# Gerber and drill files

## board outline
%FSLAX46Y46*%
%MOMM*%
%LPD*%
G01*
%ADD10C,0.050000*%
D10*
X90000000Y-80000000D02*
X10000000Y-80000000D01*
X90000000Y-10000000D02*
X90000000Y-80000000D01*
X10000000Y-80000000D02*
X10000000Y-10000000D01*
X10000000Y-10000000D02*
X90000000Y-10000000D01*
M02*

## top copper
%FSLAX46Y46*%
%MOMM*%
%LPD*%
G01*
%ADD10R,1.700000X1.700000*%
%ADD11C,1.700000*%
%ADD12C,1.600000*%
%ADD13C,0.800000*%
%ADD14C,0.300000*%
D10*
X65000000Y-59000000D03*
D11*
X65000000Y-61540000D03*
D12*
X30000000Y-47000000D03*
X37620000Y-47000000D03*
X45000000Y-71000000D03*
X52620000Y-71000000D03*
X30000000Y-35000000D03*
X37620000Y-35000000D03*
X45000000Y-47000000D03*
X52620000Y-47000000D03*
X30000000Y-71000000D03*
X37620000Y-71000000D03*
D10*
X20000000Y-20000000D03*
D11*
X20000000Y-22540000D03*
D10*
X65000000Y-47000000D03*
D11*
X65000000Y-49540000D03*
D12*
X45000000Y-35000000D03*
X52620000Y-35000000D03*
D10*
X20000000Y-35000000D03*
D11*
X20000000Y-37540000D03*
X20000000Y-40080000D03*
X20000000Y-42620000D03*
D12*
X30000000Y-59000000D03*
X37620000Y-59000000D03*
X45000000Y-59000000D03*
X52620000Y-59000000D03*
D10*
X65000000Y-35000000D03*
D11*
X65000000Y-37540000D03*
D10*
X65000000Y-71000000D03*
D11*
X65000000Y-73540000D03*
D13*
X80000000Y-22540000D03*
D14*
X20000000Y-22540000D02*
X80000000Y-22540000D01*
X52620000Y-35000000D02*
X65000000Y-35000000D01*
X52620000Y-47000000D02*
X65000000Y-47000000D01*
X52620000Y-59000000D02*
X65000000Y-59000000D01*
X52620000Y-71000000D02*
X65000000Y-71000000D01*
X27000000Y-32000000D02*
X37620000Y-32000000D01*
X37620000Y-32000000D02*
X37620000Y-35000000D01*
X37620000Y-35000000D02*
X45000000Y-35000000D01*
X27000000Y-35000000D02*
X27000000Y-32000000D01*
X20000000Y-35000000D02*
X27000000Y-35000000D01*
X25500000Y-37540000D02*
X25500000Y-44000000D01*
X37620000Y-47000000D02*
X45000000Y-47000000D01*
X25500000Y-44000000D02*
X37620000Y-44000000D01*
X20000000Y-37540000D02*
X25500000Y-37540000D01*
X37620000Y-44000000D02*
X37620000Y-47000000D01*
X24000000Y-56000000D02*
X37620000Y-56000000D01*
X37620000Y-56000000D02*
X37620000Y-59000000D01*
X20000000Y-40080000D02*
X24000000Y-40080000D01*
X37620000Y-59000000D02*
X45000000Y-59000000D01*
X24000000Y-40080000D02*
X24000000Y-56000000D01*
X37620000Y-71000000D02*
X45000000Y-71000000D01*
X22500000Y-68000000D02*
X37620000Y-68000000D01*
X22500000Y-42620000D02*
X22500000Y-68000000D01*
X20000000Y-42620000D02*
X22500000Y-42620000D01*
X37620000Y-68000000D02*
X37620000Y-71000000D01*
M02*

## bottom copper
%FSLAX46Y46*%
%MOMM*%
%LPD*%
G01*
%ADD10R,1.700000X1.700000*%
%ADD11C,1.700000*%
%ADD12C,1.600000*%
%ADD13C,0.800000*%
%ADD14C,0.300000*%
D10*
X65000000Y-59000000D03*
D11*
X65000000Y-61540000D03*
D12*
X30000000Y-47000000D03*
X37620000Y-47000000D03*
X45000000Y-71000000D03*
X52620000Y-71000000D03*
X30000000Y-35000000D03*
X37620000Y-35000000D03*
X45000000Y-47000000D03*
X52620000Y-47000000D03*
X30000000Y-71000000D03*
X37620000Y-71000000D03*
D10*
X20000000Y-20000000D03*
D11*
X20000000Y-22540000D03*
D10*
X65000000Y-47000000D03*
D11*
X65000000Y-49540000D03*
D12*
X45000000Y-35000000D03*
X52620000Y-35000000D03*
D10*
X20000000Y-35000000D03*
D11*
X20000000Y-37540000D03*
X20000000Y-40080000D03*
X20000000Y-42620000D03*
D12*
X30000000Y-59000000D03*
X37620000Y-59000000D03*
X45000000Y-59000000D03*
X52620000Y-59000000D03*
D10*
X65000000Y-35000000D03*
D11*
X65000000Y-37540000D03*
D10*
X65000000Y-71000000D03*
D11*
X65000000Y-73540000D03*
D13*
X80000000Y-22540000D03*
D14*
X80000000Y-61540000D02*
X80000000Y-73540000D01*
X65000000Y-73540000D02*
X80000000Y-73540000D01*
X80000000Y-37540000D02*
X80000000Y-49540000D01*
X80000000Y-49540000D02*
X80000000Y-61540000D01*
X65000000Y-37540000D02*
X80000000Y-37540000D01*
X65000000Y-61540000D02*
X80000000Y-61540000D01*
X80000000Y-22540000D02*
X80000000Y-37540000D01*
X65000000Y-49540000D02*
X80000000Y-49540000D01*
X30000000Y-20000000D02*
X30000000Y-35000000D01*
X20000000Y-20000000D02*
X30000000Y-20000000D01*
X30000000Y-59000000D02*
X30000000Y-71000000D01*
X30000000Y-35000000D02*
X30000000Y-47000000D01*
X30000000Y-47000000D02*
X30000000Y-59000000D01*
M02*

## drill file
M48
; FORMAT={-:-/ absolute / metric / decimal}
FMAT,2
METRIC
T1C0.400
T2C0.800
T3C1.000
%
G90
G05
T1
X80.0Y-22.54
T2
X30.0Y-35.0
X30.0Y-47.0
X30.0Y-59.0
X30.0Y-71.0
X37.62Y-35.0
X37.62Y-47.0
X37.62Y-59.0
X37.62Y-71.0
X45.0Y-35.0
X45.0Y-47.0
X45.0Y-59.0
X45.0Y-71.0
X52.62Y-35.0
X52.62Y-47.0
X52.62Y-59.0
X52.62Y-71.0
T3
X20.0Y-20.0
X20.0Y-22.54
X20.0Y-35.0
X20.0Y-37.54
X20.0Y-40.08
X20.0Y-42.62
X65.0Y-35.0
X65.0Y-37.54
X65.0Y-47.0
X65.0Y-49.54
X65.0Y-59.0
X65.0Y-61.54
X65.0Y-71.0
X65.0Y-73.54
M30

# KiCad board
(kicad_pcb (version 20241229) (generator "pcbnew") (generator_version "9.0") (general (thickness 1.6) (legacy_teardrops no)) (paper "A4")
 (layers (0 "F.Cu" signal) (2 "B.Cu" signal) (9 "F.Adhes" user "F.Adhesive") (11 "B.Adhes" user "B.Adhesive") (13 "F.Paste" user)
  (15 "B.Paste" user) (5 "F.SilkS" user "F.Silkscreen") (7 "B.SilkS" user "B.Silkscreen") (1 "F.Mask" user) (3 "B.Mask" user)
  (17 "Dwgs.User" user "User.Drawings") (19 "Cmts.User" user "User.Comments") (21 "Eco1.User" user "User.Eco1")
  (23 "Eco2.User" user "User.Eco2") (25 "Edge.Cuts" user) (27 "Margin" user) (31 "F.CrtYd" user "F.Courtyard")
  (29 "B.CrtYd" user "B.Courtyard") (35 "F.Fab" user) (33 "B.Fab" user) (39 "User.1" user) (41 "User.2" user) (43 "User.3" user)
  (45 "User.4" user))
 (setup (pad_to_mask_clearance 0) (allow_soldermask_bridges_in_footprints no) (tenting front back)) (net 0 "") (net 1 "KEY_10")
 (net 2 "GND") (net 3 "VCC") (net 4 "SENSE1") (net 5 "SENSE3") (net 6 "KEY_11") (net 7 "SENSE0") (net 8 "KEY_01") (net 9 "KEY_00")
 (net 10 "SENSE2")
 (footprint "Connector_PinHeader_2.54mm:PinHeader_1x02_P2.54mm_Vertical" (layer "F.Cu") (at 65 59)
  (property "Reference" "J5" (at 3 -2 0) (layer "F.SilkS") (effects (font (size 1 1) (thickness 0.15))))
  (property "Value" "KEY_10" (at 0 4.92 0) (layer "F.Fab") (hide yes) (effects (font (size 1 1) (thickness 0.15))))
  (pad "1" thru_hole rect (at 0 0) (size 1.7 1.7) (drill 1) (layers "*.Cu" "*.Mask") (remove_unused_layers no) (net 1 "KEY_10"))
  (pad "2" thru_hole circle (at 0 2.54) (size 1.7 1.7) (drill 1) (layers "*.Cu" "*.Mask") (remove_unused_layers no) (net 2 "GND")))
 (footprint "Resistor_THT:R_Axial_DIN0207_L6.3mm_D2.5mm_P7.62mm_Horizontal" (layer "F.Cu") (at 30 47)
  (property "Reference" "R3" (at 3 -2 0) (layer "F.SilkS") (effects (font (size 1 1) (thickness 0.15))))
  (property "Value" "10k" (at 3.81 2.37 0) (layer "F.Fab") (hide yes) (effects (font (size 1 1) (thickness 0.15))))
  (pad "1" thru_hole circle (at 0 0) (size 1.6 1.6) (drill 0.8) (layers "*.Cu" "*.Mask") (remove_unused_layers no) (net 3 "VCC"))
  (pad "2" thru_hole circle (at 7.62 0) (size 1.6 1.6) (drill 0.8) (layers "*.Cu" "*.Mask") (remove_unused_layers no) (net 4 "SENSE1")))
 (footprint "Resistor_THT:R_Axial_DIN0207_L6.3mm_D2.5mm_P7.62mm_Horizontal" (layer "F.Cu") (at 45 71)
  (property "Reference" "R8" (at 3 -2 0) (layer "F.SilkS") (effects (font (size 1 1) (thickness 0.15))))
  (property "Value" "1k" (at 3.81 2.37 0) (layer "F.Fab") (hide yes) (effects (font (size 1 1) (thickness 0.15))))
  (pad "1" thru_hole circle (at 0 0) (size 1.6 1.6) (drill 0.8) (layers "*.Cu" "*.Mask") (remove_unused_layers no) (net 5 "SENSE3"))
  (pad "2" thru_hole circle (at 7.62 0) (size 1.6 1.6) (drill 0.8) (layers "*.Cu" "*.Mask") (remove_unused_layers no) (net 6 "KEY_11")))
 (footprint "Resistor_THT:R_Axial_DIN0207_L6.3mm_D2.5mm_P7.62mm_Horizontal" (layer "F.Cu") (at 30 35)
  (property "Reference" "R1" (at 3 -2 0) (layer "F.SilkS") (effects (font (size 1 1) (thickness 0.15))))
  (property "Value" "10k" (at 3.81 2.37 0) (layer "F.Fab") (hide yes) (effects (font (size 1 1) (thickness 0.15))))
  (pad "1" thru_hole circle (at 0 0) (size 1.6 1.6) (drill 0.8) (layers "*.Cu" "*.Mask") (remove_unused_layers no) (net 3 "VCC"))
  (pad "2" thru_hole circle (at 7.62 0) (size 1.6 1.6) (drill 0.8) (layers "*.Cu" "*.Mask") (remove_unused_layers no) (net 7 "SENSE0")))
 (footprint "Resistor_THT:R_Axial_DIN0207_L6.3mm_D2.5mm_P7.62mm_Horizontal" (layer "F.Cu") (at 45 47)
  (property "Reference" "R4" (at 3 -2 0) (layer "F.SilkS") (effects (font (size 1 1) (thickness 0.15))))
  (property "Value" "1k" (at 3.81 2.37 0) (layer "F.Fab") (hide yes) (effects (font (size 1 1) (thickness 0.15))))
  (pad "1" thru_hole circle (at 0 0) (size 1.6 1.6) (drill 0.8) (layers "*.Cu" "*.Mask") (remove_unused_layers no) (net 4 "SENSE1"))
  (pad "2" thru_hole circle (at 7.62 0) (size 1.6 1.6) (drill 0.8) (layers "*.Cu" "*.Mask") (remove_unused_layers no) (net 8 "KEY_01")))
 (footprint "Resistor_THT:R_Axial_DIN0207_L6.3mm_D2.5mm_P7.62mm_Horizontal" (layer "F.Cu") (at 30 71)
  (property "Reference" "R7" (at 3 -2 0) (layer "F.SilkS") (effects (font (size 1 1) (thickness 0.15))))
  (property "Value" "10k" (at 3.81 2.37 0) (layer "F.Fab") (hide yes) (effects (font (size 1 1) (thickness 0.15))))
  (pad "1" thru_hole circle (at 0 0) (size 1.6 1.6) (drill 0.8) (layers "*.Cu" "*.Mask") (remove_unused_layers no) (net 3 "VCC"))
  (pad "2" thru_hole circle (at 7.62 0) (size 1.6 1.6) (drill 0.8) (layers "*.Cu" "*.Mask") (remove_unused_layers no) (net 5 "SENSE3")))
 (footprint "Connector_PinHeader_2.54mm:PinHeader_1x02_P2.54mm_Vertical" (layer "F.Cu") (at 20 20)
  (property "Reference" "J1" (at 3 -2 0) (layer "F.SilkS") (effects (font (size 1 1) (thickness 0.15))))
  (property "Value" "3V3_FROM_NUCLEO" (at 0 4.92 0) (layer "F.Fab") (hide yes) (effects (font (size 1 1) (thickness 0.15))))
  (pad "1" thru_hole rect (at 0 0) (size 1.7 1.7) (drill 1) (layers "*.Cu" "*.Mask") (remove_unused_layers no) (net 3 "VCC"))
  (pad "2" thru_hole circle (at 0 2.54) (size 1.7 1.7) (drill 1) (layers "*.Cu" "*.Mask") (remove_unused_layers no) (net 2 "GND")))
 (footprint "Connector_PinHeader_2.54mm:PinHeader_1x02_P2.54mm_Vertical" (layer "F.Cu") (at 65 47)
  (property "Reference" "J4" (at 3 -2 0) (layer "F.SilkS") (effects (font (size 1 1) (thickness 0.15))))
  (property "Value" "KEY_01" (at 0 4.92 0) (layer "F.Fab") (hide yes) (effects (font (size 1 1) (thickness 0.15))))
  (pad "1" thru_hole rect (at 0 0) (size 1.7 1.7) (drill 1) (layers "*.Cu" "*.Mask") (remove_unused_layers no) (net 8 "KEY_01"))
  (pad "2" thru_hole circle (at 0 2.54) (size 1.7 1.7) (drill 1) (layers "*.Cu" "*.Mask") (remove_unused_layers no) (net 2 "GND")))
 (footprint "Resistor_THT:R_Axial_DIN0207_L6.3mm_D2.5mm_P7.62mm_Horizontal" (layer "F.Cu") (at 45 35)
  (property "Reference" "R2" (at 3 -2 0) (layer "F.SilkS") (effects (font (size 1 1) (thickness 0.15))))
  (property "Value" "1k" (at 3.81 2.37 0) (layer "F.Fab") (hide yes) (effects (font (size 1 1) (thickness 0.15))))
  (pad "1" thru_hole circle (at 0 0) (size 1.6 1.6) (drill 0.8) (layers "*.Cu" "*.Mask") (remove_unused_layers no) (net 7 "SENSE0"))
  (pad "2" thru_hole circle (at 7.62 0) (size 1.6 1.6) (drill 0.8) (layers "*.Cu" "*.Mask") (remove_unused_layers no) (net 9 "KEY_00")))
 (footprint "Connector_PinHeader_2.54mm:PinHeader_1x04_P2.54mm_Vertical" (layer "F.Cu") (at 20 35)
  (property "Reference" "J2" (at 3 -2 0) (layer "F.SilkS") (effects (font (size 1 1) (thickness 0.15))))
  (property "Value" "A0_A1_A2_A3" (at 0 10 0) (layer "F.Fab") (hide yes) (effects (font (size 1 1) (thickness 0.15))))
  (pad "1" thru_hole rect (at 0 0) (size 1.7 1.7) (drill 1) (layers "*.Cu" "*.Mask") (remove_unused_layers no) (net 7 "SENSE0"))
  (pad "2" thru_hole circle (at 0 2.54) (size 1.7 1.7) (drill 1) (layers "*.Cu" "*.Mask") (remove_unused_layers no) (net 4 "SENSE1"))
  (pad "3" thru_hole circle (at 0 5.08) (size 1.7 1.7) (drill 1) (layers "*.Cu" "*.Mask") (remove_unused_layers no) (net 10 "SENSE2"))
  (pad "4" thru_hole circle (at 0 7.62) (size 1.7 1.7) (drill 1) (layers "*.Cu" "*.Mask") (remove_unused_layers no) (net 5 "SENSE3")))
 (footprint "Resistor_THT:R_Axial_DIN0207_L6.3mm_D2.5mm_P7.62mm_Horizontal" (layer "F.Cu") (at 30 59)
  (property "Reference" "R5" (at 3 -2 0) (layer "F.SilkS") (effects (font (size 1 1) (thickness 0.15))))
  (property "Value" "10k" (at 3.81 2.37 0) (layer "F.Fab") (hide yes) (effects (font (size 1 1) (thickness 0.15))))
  (pad "1" thru_hole circle (at 0 0) (size 1.6 1.6) (drill 0.8) (layers "*.Cu" "*.Mask") (remove_unused_layers no) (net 3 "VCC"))
  (pad "2" thru_hole circle (at 7.62 0) (size 1.6 1.6) (drill 0.8) (layers "*.Cu" "*.Mask") (remove_unused_layers no) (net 10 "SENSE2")))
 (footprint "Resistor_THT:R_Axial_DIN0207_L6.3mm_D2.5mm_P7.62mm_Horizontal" (layer "F.Cu") (at 45 59)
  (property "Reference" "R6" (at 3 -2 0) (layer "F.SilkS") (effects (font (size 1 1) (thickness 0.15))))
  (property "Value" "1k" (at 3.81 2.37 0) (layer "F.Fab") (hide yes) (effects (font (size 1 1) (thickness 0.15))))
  (pad "1" thru_hole circle (at 0 0) (size 1.6 1.6) (drill 0.8) (layers "*.Cu" "*.Mask") (remove_unused_layers no) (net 10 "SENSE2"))
  (pad "2" thru_hole circle (at 7.62 0) (size 1.6 1.6) (drill 0.8) (layers "*.Cu" "*.Mask") (remove_unused_layers no) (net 1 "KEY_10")))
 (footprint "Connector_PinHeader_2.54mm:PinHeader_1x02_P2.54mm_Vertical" (layer "F.Cu") (at 65 35)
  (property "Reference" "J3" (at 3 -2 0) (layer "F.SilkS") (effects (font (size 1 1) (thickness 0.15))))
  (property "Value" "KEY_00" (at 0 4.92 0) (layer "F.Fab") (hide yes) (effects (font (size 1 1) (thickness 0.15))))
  (pad "1" thru_hole rect (at 0 0) (size 1.7 1.7) (drill 1) (layers "*.Cu" "*.Mask") (remove_unused_layers no) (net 9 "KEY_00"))
  (pad "2" thru_hole circle (at 0 2.54) (size 1.7 1.7) (drill 1) (layers "*.Cu" "*.Mask") (remove_unused_layers no) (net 2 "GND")))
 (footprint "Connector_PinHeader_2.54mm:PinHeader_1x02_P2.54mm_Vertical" (layer "F.Cu") (at 65 71)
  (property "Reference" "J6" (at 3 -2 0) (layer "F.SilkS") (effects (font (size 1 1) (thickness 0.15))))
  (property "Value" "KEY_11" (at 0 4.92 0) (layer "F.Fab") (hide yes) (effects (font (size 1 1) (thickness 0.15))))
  (pad "1" thru_hole rect (at 0 0) (size 1.7 1.7) (drill 1) (layers "*.Cu" "*.Mask") (remove_unused_layers no) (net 6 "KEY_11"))
  (pad "2" thru_hole circle (at 0 2.54) (size 1.7 1.7) (drill 1) (layers "*.Cu" "*.Mask") (remove_unused_layers no) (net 2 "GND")))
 (gr_line (start 90 80) (end 10 80) (stroke (width 0.05) (type default)) (layer "Edge.Cuts"))
 (gr_line (start 90 10) (end 90 80) (stroke (width 0.05) (type default)) (layer "Edge.Cuts"))
 (gr_line (start 10 80) (end 10 10) (stroke (width 0.05) (type default)) (layer "Edge.Cuts"))
 (gr_line (start 10 10) (end 90 10) (stroke (width 0.05) (type default)) (layer "Edge.Cuts"))
 (segment (start 20 22.54) (end 80 22.54) (width 0.3) (layer "F.Cu") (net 2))
 (via (at 80 22.54) (size 0.8) (drill 0.4) (layers "F.Cu" "B.Cu") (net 2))
 (segment (start 80 61.54) (end 80 73.54) (width 0.3) (layer "B.Cu") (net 2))
 (segment (start 65 73.54) (end 80 73.54) (width 0.3) (layer "B.Cu") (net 2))
 (segment (start 80 37.54) (end 80 49.54) (width 0.3) (layer "B.Cu") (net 2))
 (segment (start 80 49.54) (end 80 61.54) (width 0.3) (layer "B.Cu") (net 2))
 (segment (start 65 37.54) (end 80 37.54) (width 0.3) (layer "B.Cu") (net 2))
 (segment (start 65 61.54) (end 80 61.54) (width 0.3) (layer "B.Cu") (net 2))
 (segment (start 80 22.54) (end 80 37.54) (width 0.3) (layer "B.Cu") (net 2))
 (segment (start 65 49.54) (end 80 49.54) (width 0.3) (layer "B.Cu") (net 2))
 (segment (start 52.62 35) (end 65 35) (width 0.3) (layer "F.Cu") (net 9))
 (segment (start 52.62 47) (end 65 47) (width 0.3) (layer "F.Cu") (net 8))
 (segment (start 52.62 59) (end 65 59) (width 0.3) (layer "F.Cu") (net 1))
 (segment (start 52.62 71) (end 65 71) (width 0.3) (layer "F.Cu") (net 6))
 (segment (start 27 32) (end 37.62 32) (width 0.3) (layer "F.Cu") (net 7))
 (segment (start 37.62 32) (end 37.62 35) (width 0.3) (layer "F.Cu") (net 7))
 (segment (start 37.62 35) (end 45 35) (width 0.3) (layer "F.Cu") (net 7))
 (segment (start 27 35) (end 27 32) (width 0.3) (layer "F.Cu") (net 7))
 (segment (start 20 35) (end 27 35) (width 0.3) (layer "F.Cu") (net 7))
 (segment (start 25.5 37.54) (end 25.5 44) (width 0.3) (layer "F.Cu") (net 4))
 (segment (start 37.62 47) (end 45 47) (width 0.3) (layer "F.Cu") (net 4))
 (segment (start 25.5 44) (end 37.62 44) (width 0.3) (layer "F.Cu") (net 4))
 (segment (start 20 37.54) (end 25.5 37.54) (width 0.3) (layer "F.Cu") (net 4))
 (segment (start 37.62 44) (end 37.62 47) (width 0.3) (layer "F.Cu") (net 4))
 (segment (start 24 56) (end 37.62 56) (width 0.3) (layer "F.Cu") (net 10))
 (segment (start 37.62 56) (end 37.62 59) (width 0.3) (layer "F.Cu") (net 10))
 (segment (start 20 40.08) (end 24 40.08) (width 0.3) (layer "F.Cu") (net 10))
 (segment (start 37.62 59) (end 45 59) (width 0.3) (layer "F.Cu") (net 10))
 (segment (start 24 40.08) (end 24 56) (width 0.3) (layer "F.Cu") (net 10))
 (segment (start 37.62 71) (end 45 71) (width 0.3) (layer "F.Cu") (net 5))
 (segment (start 22.5 68) (end 37.62 68) (width 0.3) (layer "F.Cu") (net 5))
 (segment (start 22.5 42.62) (end 22.5 68) (width 0.3) (layer "F.Cu") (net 5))
 (segment (start 20 42.62) (end 22.5 42.62) (width 0.3) (layer "F.Cu") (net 5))
 (segment (start 37.62 68) (end 37.62 71) (width 0.3) (layer "F.Cu") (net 5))
 (segment (start 30 20) (end 30 35) (width 0.3) (layer "B.Cu") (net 3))
 (segment (start 20 20) (end 30 20) (width 0.3) (layer "B.Cu") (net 3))
 (segment (start 30 59) (end 30 71) (width 0.3) (layer "B.Cu") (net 3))
 (segment (start 30 35) (end 30 47) (width 0.3) (layer "B.Cu") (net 3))
 (segment (start 30 47) (end 30 59) (width 0.3) (layer "B.Cu") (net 3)))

